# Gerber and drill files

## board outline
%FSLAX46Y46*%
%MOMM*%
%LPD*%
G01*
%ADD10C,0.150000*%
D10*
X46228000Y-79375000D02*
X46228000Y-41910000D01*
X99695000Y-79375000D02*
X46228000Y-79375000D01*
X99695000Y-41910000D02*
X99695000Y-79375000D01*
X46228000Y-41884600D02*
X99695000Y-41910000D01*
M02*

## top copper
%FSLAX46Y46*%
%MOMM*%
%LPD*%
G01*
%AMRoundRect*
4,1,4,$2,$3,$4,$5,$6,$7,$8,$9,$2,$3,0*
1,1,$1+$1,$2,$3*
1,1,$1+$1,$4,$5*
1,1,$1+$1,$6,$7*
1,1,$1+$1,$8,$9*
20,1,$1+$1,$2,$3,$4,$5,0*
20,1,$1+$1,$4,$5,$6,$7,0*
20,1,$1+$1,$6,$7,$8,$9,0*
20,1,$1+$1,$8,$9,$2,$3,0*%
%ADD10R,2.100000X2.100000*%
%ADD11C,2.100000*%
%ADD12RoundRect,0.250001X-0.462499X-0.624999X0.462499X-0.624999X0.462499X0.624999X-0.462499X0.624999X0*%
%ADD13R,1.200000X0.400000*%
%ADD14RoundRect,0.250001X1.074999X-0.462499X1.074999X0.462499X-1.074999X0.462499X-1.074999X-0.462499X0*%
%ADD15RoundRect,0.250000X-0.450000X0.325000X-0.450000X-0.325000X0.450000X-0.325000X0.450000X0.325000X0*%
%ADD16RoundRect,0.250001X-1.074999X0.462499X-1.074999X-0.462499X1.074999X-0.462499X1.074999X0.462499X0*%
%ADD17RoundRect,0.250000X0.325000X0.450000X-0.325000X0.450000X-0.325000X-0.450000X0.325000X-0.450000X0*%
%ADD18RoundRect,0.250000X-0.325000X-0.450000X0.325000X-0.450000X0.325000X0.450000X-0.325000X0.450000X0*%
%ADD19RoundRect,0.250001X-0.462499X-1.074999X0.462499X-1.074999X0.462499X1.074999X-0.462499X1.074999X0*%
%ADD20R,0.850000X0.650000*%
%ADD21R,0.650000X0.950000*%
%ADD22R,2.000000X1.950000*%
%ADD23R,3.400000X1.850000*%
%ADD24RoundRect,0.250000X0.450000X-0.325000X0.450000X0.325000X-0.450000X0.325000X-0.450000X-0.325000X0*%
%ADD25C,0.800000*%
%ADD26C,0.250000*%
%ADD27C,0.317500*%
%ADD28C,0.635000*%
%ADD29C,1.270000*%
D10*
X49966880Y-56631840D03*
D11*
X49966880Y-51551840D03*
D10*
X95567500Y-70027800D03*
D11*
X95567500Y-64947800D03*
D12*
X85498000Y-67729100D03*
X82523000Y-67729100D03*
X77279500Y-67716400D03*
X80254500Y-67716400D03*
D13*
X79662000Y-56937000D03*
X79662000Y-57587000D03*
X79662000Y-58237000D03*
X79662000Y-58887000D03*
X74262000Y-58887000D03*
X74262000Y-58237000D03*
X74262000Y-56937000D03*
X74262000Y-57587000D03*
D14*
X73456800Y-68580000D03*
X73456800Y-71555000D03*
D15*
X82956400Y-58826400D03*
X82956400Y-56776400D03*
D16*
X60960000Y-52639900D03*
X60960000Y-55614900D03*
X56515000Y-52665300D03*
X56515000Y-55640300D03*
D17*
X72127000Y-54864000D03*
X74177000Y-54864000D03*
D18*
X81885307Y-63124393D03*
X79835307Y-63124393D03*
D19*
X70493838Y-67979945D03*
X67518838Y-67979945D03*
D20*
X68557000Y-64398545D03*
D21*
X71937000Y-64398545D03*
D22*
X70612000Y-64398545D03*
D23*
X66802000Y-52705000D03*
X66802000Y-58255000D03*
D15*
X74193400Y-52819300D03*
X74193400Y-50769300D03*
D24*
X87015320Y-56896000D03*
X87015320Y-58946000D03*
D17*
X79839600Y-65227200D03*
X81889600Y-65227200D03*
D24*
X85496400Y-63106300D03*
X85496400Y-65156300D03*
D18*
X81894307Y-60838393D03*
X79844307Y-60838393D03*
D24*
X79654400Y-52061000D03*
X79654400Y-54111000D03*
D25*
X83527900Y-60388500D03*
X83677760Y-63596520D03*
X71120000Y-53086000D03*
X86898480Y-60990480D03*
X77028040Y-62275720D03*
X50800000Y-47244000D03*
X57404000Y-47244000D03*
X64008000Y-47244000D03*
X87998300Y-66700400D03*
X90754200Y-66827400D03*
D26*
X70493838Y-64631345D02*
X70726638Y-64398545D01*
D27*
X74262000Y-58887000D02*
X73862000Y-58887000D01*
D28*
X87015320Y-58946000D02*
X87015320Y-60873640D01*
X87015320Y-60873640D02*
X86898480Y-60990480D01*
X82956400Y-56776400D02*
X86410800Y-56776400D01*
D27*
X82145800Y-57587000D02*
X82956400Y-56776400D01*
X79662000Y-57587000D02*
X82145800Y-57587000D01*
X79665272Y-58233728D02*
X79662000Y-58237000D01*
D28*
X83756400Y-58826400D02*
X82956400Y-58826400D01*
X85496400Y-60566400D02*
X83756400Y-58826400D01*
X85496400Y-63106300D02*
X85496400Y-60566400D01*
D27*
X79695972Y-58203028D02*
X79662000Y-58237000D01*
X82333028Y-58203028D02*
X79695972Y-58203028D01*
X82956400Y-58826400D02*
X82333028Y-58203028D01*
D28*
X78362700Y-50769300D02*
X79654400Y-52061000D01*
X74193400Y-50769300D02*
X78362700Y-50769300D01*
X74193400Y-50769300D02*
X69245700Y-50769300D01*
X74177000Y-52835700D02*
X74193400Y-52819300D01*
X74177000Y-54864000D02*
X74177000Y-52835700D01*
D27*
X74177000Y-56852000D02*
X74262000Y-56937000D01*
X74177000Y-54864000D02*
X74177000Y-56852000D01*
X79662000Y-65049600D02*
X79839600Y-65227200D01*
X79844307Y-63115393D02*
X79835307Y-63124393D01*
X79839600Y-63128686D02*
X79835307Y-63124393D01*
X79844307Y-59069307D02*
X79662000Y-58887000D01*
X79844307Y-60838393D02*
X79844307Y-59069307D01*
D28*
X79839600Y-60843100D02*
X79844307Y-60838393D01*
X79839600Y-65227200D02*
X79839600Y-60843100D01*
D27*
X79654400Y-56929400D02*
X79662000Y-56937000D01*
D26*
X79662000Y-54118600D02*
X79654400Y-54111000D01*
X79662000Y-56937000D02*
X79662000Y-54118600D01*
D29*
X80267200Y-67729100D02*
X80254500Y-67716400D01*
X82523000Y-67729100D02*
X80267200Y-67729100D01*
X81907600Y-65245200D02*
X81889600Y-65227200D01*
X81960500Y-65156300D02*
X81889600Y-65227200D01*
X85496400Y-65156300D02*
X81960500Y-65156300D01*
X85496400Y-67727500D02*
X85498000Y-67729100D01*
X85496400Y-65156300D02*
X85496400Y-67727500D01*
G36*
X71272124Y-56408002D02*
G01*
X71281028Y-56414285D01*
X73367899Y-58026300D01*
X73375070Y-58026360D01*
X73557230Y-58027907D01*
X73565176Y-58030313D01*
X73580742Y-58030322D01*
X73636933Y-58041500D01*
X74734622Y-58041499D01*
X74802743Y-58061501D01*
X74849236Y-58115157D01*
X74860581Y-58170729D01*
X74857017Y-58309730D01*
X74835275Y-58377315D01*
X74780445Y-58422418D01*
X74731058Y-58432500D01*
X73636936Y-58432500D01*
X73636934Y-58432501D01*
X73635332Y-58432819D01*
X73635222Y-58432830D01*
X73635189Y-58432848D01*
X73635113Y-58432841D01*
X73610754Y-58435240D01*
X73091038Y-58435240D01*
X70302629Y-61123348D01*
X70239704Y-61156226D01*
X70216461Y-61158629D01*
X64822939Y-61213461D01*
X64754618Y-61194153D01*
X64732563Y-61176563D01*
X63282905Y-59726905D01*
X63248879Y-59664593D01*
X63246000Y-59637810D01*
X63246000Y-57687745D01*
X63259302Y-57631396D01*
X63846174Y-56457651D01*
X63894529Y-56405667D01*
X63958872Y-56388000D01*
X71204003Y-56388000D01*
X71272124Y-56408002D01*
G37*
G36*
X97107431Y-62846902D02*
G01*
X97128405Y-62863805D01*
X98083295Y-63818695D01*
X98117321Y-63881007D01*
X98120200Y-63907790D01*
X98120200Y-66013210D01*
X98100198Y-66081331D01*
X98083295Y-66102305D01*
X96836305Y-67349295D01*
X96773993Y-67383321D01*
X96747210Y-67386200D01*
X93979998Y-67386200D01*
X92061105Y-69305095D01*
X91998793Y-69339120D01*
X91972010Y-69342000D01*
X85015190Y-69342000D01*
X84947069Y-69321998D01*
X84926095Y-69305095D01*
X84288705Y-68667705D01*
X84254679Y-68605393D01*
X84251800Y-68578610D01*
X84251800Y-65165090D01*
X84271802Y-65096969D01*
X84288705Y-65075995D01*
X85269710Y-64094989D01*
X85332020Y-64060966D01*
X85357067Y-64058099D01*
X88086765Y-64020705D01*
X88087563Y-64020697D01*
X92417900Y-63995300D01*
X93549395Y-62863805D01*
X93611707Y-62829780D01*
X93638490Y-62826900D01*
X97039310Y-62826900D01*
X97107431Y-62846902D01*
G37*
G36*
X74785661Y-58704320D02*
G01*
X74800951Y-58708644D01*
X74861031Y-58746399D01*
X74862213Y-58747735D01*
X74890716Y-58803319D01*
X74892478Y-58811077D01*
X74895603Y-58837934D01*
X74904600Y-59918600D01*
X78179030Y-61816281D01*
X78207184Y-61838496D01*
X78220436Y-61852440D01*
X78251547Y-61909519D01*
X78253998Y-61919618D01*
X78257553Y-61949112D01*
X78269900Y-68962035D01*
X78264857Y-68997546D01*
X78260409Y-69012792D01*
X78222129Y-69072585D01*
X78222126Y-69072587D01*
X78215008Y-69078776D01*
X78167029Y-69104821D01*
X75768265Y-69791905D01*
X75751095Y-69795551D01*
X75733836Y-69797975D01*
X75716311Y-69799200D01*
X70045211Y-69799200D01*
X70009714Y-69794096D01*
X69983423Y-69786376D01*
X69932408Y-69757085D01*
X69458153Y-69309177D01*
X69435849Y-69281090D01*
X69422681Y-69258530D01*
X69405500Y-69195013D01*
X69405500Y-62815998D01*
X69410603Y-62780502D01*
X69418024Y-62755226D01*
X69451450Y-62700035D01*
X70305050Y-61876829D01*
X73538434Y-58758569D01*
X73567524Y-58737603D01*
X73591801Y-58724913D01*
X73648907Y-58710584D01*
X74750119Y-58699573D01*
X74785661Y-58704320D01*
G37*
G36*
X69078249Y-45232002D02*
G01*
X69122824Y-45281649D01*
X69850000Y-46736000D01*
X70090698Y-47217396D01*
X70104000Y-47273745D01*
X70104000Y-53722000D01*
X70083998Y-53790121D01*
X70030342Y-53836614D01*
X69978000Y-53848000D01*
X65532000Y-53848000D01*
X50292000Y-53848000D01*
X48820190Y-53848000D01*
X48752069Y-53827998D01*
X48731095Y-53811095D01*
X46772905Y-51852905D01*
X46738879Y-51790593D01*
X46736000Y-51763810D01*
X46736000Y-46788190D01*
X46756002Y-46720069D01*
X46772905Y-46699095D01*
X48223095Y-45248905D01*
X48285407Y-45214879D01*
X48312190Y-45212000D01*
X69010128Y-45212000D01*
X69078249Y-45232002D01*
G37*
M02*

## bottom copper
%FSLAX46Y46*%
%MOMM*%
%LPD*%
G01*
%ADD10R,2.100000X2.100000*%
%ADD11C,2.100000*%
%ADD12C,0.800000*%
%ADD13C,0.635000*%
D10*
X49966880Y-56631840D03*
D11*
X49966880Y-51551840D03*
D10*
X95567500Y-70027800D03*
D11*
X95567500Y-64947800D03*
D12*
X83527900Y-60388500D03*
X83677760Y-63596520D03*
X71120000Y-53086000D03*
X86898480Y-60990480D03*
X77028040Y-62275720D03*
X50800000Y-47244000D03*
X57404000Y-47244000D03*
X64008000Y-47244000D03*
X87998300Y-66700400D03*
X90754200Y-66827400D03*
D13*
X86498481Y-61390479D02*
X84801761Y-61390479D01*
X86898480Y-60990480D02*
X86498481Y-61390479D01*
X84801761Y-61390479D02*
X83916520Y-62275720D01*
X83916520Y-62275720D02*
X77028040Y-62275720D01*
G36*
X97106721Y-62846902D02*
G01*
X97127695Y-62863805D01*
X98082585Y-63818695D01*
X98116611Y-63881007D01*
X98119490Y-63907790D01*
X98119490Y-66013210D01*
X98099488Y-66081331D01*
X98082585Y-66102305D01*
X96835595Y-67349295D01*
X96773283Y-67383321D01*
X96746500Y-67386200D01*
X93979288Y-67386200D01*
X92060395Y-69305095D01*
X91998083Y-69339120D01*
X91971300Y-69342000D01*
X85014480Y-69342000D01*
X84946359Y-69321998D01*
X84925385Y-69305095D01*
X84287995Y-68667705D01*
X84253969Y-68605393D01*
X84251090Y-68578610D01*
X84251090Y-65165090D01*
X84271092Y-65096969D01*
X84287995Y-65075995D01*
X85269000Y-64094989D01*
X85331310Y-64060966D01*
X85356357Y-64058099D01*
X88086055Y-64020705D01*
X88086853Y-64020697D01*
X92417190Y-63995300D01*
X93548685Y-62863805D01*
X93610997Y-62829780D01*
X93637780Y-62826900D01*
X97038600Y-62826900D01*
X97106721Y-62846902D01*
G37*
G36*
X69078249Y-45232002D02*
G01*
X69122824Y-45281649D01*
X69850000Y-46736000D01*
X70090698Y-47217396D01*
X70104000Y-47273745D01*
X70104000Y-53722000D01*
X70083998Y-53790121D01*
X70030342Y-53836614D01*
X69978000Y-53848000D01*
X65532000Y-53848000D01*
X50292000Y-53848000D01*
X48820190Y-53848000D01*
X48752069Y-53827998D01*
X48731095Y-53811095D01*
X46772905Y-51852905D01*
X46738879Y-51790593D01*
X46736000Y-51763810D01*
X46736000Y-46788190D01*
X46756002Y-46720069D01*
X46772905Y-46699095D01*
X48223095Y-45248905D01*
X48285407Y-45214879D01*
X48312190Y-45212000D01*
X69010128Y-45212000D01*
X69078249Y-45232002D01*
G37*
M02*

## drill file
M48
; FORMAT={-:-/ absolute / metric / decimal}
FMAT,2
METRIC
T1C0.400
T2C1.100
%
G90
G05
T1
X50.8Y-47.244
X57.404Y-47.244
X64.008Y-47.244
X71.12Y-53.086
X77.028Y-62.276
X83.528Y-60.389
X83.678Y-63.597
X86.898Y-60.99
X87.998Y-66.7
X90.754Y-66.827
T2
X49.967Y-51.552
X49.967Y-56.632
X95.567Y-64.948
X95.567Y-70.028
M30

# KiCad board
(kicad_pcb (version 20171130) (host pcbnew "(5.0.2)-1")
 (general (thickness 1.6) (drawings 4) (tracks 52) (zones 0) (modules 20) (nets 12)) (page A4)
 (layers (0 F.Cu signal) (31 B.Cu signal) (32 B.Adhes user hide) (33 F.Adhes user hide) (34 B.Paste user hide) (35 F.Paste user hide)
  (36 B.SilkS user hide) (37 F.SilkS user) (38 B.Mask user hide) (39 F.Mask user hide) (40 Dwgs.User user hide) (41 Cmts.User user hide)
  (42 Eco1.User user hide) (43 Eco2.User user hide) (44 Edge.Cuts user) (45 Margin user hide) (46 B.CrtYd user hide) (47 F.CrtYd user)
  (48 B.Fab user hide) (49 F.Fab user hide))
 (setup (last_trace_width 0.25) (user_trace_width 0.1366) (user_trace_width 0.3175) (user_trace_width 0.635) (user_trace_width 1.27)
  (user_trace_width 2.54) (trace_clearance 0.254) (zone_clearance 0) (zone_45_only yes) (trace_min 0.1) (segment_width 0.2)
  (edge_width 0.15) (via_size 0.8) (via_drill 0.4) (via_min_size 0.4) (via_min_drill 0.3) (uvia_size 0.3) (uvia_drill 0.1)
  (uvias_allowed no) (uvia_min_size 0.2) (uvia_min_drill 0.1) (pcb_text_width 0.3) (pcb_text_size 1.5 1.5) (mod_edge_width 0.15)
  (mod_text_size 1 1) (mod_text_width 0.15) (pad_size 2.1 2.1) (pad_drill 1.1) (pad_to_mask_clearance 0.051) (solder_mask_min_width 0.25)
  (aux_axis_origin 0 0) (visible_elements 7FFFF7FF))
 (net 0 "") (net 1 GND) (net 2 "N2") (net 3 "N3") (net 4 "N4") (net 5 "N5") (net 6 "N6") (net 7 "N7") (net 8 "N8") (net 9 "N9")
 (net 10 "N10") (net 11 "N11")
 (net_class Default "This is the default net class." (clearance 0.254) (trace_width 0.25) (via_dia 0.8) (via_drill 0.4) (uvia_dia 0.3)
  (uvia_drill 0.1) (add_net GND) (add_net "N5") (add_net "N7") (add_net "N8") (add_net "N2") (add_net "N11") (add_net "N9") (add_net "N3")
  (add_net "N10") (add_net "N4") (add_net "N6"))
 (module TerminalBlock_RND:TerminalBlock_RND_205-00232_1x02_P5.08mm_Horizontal (layer F.Cu) (at 49.96688 56.63184 90)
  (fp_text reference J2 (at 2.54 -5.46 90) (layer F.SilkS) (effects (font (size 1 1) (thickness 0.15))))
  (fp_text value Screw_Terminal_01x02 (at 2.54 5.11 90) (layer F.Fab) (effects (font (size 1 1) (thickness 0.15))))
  (pad 1 thru_hole rect (at 0 0 90) (size 2.1 2.1) (drill 1.1) (layers *.Cu *.Mask) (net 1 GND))
  (pad 2 thru_hole circle (at 5.08 0 90) (size 2.1 2.1) (drill 1.1) (layers *.Cu *.Mask) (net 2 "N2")))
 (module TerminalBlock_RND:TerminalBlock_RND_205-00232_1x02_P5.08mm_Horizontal (layer F.Cu) (at 95.5675 70.0278 90)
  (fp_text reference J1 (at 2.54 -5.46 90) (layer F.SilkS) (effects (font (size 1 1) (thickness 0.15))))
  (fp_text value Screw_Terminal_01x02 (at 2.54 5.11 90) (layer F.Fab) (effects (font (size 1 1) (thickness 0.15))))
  (pad 1 thru_hole rect (at 0 0 90) (size 2.1 2.1) (drill 1.1) (layers *.Cu *.Mask) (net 1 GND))
  (pad 2 thru_hole circle (at 5.08 0 90) (size 2.1 2.1) (drill 1.1) (layers *.Cu *.Mask) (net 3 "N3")))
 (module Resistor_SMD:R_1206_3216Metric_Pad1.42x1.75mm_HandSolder (layer F.Cu) (at 84.0105 67.7291)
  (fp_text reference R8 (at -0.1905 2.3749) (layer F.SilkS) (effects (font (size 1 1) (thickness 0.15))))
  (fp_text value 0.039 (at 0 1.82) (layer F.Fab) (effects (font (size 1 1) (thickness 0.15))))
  (pad 2 smd roundrect (at 1.4875 0) (size 1.425 1.75) (layers F.Cu F.Paste F.Mask) (roundrect_rratio 0.175439) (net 3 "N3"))
  (pad 1 smd roundrect (at -1.4875 0) (size 1.425 1.75) (layers F.Cu F.Paste F.Mask) (roundrect_rratio 0.175439) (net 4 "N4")))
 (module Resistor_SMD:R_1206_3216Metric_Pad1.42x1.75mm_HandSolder (layer F.Cu) (at 78.767 67.7164)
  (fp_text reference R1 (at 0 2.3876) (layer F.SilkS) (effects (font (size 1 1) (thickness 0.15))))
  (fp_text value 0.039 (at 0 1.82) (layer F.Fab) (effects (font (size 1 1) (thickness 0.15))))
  (pad 1 smd roundrect (at -1.4875 0) (size 1.425 1.75) (layers F.Cu F.Paste F.Mask) (roundrect_rratio 0.175439) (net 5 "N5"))
  (pad 2 smd roundrect (at 1.4875 0) (size 1.425 1.75) (layers F.Cu F.Paste F.Mask) (roundrect_rratio 0.175439) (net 4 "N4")))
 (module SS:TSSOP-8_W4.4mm (layer F.Cu) (at 76.962 57.912)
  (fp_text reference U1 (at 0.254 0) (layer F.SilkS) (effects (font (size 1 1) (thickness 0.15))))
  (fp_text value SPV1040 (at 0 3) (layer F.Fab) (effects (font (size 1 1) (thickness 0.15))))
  (pad 8 smd rect (at 2.7 -0.975) (size 1.2 0.4) (layers F.Cu F.Paste F.Mask) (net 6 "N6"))
  (pad 7 smd rect (at 2.7 -0.325) (size 1.2 0.4) (layers F.Cu F.Paste F.Mask) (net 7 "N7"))
  (pad 6 smd rect (at 2.7 0.325) (size 1.2 0.4) (layers F.Cu F.Paste F.Mask) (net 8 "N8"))
  (pad 5 smd rect (at 2.7 0.975) (size 1.2 0.4) (layers F.Cu F.Paste F.Mask) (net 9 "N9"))
  (pad 4 smd rect (at -2.7 0.975) (size 1.2 0.4) (layers F.Cu F.Paste F.Mask) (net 5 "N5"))
  (pad 3 smd rect (at -2.7 0.325) (size 1.2 0.4) (layers F.Cu F.Paste F.Mask) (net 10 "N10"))
  (pad 1 smd rect (at -2.7 -0.975) (size 1.2 0.4) (layers F.Cu F.Paste F.Mask) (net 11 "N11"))
  (pad 2 smd rect (at -2.7 -0.325) (size 1.2 0.4) (layers F.Cu F.Paste F.Mask) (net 1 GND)))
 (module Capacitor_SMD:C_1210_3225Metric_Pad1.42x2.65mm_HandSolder (layer F.Cu) (at 73.4568 70.0675 90)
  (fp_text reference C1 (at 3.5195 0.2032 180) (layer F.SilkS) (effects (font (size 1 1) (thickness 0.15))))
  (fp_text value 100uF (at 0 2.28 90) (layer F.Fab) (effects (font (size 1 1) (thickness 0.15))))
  (pad 2 smd roundrect (at 1.4875 0 90) (size 1.425 2.65) (layers F.Cu F.Paste F.Mask) (roundrect_rratio 0.175439) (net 5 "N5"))
  (pad 1 smd roundrect (at -1.4875 0 90) (size 1.425 2.65) (layers F.Cu F.Paste F.Mask) (roundrect_rratio 0.175439) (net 1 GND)))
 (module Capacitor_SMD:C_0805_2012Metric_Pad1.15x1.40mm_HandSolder (layer F.Cu) (at 82.9564 57.8014 270)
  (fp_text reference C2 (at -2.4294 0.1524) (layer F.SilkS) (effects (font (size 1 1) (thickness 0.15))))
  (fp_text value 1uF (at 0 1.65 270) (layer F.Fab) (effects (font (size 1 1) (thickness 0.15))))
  (pad 2 smd roundrect (at 1.025 0 270) (size 1.15 1.4) (layers F.Cu F.Paste F.Mask) (roundrect_rratio 0.217391) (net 8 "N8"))
  (pad 1 smd roundrect (at -1.025 0 270) (size 1.15 1.4) (layers F.Cu F.Paste F.Mask) (roundrect_rratio 0.217391) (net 7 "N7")))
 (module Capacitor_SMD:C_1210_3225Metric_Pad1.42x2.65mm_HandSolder (layer F.Cu) (at 60.96 54.1274 270)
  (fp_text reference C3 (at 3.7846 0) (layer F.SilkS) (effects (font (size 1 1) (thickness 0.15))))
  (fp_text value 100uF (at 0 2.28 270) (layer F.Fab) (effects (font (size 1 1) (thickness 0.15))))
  (pad 1 smd roundrect (at -1.4875 0 270) (size 1.425 2.65) (layers F.Cu F.Paste F.Mask) (roundrect_rratio 0.175439) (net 2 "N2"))
  (pad 2 smd roundrect (at 1.4875 0 270) (size 1.425 2.65) (layers F.Cu F.Paste F.Mask) (roundrect_rratio 0.175439) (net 1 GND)))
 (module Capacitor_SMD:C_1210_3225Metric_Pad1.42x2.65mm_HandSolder (layer F.Cu) (at 56.515 54.1528 270)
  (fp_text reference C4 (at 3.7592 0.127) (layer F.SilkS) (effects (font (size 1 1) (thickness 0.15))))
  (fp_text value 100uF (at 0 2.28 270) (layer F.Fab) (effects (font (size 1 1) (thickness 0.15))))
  (pad 1 smd roundrect (at -1.4875 0 270) (size 1.425 2.65) (layers F.Cu F.Paste F.Mask) (roundrect_rratio 0.175439) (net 2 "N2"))
  (pad 2 smd roundrect (at 1.4875 0 270) (size 1.425 2.65) (layers F.Cu F.Paste F.Mask) (roundrect_rratio 0.175439) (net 1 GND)))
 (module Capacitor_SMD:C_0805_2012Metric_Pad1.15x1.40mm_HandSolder (layer F.Cu) (at 73.152 54.864 180)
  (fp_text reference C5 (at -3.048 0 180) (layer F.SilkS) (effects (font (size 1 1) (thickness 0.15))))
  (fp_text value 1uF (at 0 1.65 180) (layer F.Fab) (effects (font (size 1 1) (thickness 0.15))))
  (pad 2 smd roundrect (at 1.025 0 180) (size 1.15 1.4) (layers F.Cu F.Paste F.Mask) (roundrect_rratio 0.217391) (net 1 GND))
  (pad 1 smd roundrect (at -1.025 0 180) (size 1.15 1.4) (layers F.Cu F.Paste F.Mask) (roundrect_rratio 0.217391) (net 11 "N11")))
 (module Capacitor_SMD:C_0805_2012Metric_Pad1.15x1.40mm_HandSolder (layer F.Cu) (at 80.860307 63.124393)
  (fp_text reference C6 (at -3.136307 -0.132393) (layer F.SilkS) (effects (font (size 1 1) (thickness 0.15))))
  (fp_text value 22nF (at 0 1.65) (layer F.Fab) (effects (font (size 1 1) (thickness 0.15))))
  (pad 2 smd roundrect (at 1.025 0) (size 1.15 1.4) (layers F.Cu F.Paste F.Mask) (roundrect_rratio 0.217391) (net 1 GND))
  (pad 1 smd roundrect (at -1.025 0) (size 1.15 1.4) (layers F.Cu F.Paste F.Mask) (roundrect_rratio 0.217391) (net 9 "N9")))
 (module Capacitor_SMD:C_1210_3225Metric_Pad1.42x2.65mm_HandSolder (layer F.Cu) (at 69.006338 67.979945)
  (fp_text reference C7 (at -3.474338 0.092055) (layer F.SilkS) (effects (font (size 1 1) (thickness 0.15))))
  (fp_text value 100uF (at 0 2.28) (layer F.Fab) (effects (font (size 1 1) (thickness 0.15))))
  (pad 2 smd roundrect (at 1.4875 0) (size 1.425 2.65) (layers F.Cu F.Paste F.Mask) (roundrect_rratio 0.175439) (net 5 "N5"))
  (pad 1 smd roundrect (at -1.4875 0) (size 1.425 2.65) (layers F.Cu F.Paste F.Mask) (roundrect_rratio 0.175439) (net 1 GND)))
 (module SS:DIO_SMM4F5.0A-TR (layer F.Cu) (at 70.197 64.398545 180)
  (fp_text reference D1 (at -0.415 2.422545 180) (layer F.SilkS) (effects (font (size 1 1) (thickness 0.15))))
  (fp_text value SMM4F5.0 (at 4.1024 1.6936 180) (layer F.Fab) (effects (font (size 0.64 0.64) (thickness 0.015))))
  (pad 2 smd rect (at 1.64 0 180) (size 0.85 0.65) (layers F.Cu F.Paste F.Mask) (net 1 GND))
  (pad 1 smd rect (at -1.74 0 180) (size 0.65 0.95) (layers F.Cu F.Paste F.Mask) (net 5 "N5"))
  (pad 1 smd rect (at -0.415 0 180) (size 2 1.95) (layers F.Cu F.Paste F.Mask) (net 5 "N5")))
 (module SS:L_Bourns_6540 (layer F.Cu) (at 66.802 52.705 270)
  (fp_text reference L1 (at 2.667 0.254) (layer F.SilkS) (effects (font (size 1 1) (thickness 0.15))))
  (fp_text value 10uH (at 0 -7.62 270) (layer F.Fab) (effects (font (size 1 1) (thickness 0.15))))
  (pad 1 smd rect (at 0 0 270) (size 1.85 3.4) (layers F.Cu F.Paste F.Mask) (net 2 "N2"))
  (pad 2 smd rect (at 5.55 0 270) (size 1.85 3.4) (layers F.Cu F.Paste F.Mask) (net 10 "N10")))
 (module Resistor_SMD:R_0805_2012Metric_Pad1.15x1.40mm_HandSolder (layer F.Cu) (at 74.1934 51.7943 270)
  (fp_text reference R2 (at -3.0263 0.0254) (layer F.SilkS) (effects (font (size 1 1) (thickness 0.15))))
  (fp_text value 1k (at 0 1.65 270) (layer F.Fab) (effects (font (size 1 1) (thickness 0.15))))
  (pad 2 smd roundrect (at 1.025 0 270) (size 1.15 1.4) (layers F.Cu F.Paste F.Mask) (roundrect_rratio 0.217391) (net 11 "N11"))
  (pad 1 smd roundrect (at -1.025 0 270) (size 1.15 1.4) (layers F.Cu F.Paste F.Mask) (roundrect_rratio 0.217391) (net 2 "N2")))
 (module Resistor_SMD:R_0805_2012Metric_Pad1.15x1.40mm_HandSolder (layer F.Cu) (at 87.01532 57.921 90)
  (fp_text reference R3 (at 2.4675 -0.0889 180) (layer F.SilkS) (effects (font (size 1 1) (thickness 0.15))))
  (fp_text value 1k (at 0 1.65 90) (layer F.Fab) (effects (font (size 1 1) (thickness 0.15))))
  (pad 2 smd roundrect (at 1.025 0 90) (size 1.15 1.4) (layers F.Cu F.Paste F.Mask) (roundrect_rratio 0.217391) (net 7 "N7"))
  (pad 1 smd roundrect (at -1.025 0 90) (size 1.15 1.4) (layers F.Cu F.Paste F.Mask) (roundrect_rratio 0.217391) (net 5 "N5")))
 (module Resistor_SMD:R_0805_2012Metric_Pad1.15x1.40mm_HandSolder (layer F.Cu) (at 80.8646 65.2272 180)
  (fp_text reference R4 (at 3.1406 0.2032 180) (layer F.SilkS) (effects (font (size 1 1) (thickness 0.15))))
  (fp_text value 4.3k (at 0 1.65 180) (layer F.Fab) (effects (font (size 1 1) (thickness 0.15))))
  (pad 2 smd roundrect (at 1.025 0 180) (size 1.15 1.4) (layers F.Cu F.Paste F.Mask) (roundrect_rratio 0.217391) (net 9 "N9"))
  (pad 1 smd roundrect (at -1.025 0 180) (size 1.15 1.4) (layers F.Cu F.Paste F.Mask) (roundrect_rratio 0.217391) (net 3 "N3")))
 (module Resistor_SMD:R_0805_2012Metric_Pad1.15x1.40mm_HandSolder (layer F.Cu) (at 85.4964 64.1313 90)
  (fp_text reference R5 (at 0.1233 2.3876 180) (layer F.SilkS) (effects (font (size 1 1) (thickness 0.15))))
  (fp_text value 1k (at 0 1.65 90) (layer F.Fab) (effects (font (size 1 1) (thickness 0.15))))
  (pad 2 smd roundrect (at 1.025 0 90) (size 1.15 1.4) (layers F.Cu F.Paste F.Mask) (roundrect_rratio 0.217391) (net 8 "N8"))
  (pad 1 smd roundrect (at -1.025 0 90) (size 1.15 1.4) (layers F.Cu F.Paste F.Mask) (roundrect_rratio 0.217391) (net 3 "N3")))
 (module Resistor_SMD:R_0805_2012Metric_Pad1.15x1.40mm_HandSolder (layer F.Cu) (at 80.869307 60.838393)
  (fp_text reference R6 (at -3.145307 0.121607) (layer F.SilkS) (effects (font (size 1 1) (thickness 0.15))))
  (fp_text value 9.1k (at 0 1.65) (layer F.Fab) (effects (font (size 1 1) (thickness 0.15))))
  (pad 2 smd roundrect (at 1.025 0) (size 1.15 1.4) (layers F.Cu F.Paste F.Mask) (roundrect_rratio 0.217391) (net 1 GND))
  (pad 1 smd roundrect (at -1.025 0) (size 1.15 1.4) (layers F.Cu F.Paste F.Mask) (roundrect_rratio 0.217391) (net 9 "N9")))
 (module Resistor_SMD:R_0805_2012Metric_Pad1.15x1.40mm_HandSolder (layer F.Cu) (at 79.6544 53.086 90)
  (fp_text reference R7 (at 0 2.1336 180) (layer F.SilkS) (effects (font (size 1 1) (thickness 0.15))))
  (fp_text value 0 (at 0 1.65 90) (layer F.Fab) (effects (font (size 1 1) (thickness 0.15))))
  (pad 2 smd roundrect (at 1.025 0 90) (size 1.15 1.4) (layers F.Cu F.Paste F.Mask) (roundrect_rratio 0.217391) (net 2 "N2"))
  (pad 1 smd roundrect (at -1.025 0 90) (size 1.15 1.4) (layers F.Cu F.Paste F.Mask) (roundrect_rratio 0.217391) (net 6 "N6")))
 (gr_line (start 46.228 79.375) (end 46.228 41.91) (layer Edge.Cuts) (width 0.15))
 (gr_line (start 99.695 79.375) (end 46.228 79.375) (layer Edge.Cuts) (width 0.15))
 (gr_line (start 99.695 41.91) (end 99.695 79.375) (layer Edge.Cuts) (width 0.15))
 (gr_line (start 46.228 41.8846) (end 99.695 41.91) (layer Edge.Cuts) (width 0.15))
 (via (at 83.5279 60.3885) (size 0.8) (drill 0.4) (layers F.Cu B.Cu) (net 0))
 (via (at 83.67776 63.59652) (size 0.8) (drill 0.4) (layers F.Cu B.Cu) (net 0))
 (via (at 71.12 53.086) (size 0.8) (drill 0.4) (layers F.Cu B.Cu) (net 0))
 (segment (start 70.493838 64.631345) (end 70.726638 64.398545) (width 0.25) (layer F.Cu) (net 5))
 (segment (start 74.262 58.887) (end 73.862 58.887) (width 0.3175) (layer F.Cu) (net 5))
 (via (at 86.89848 60.99048) (size 0.8) (drill 0.4) (layers F.Cu B.Cu) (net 5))
 (segment (start 87.01532 58.946) (end 87.01532 60.87364) (width 0.635) (layer F.Cu) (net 5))
 (segment (start 87.01532 60.87364) (end 86.89848 60.99048) (width 0.635) (layer F.Cu) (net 5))
 (segment (start 86.498481 61.390479) (end 84.801761 61.390479) (width 0.635) (layer B.Cu) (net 5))
 (segment (start 86.89848 60.99048) (end 86.498481 61.390479) (width 0.635) (layer B.Cu) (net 5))
 (segment (start 84.801761 61.390479) (end 83.91652 62.27572) (width 0.635) (layer B.Cu) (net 5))
 (via (at 77.02804 62.27572) (size 0.8) (drill 0.4) (layers F.Cu B.Cu) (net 5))
 (segment (start 83.91652 62.27572) (end 77.02804 62.27572) (width 0.635) (layer B.Cu) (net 5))
 (segment (start 82.9564 56.7764) (end 86.4108 56.7764) (width 0.635) (layer F.Cu) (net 7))
 (segment (start 82.1458 57.587) (end 82.9564 56.7764) (width 0.3175) (layer F.Cu) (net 7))
 (segment (start 79.662 57.587) (end 82.1458 57.587) (width 0.3175) (layer F.Cu) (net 7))
 (segment (start 79.665272 58.233728) (end 79.662 58.237) (width 0.3175) (layer F.Cu) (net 8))
 (segment (start 83.7564 58.8264) (end 82.9564 58.8264) (width 0.635) (layer F.Cu) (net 8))
 (segment (start 85.4964 60.5664) (end 83.7564 58.8264) (width 0.635) (layer F.Cu) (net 8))
 (segment (start 85.4964 63.1063) (end 85.4964 60.5664) (width 0.635) (layer F.Cu) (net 8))
 (segment (start 79.695972 58.203028) (end 79.662 58.237) (width 0.3175) (layer F.Cu) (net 8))
 (segment (start 82.333028 58.203028) (end 79.695972 58.203028) (width 0.3175) (layer F.Cu) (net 8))
 (segment (start 82.9564 58.8264) (end 82.333028 58.203028) (width 0.3175) (layer F.Cu) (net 8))
 (via (at 50.8 47.244) (size 0.8) (drill 0.4) (layers F.Cu B.Cu) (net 2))
 (via (at 57.404 47.244) (size 0.8) (drill 0.4) (layers F.Cu B.Cu) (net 2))
 (via (at 64.008 47.244) (size 0.8) (drill 0.4) (layers F.Cu B.Cu) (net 2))
 (segment (start 78.3627 50.7693) (end 79.6544 52.061) (width 0.635) (layer F.Cu) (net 2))
 (segment (start 74.1934 50.7693) (end 78.3627 50.7693) (width 0.635) (layer F.Cu) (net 2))
 (segment (start 74.1934 50.7693) (end 69.2457 50.7693) (width 0.635) (layer F.Cu) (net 2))
 (segment (start 74.177 52.8357) (end 74.1934 52.8193) (width 0.635) (layer F.Cu) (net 11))
 (segment (start 74.177 54.864) (end 74.177 52.8357) (width 0.635) (layer F.Cu) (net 11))
 (segment (start 74.177 56.852) (end 74.262 56.937) (width 0.3175) (layer F.Cu) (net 11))
 (segment (start 74.177 54.864) (end 74.177 56.852) (width 0.3175) (layer F.Cu) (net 11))
 (segment (start 79.662 65.0496) (end 79.8396 65.2272) (width 0.3175) (layer F.Cu) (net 9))
 (segment (start 79.844307 63.115393) (end 79.835307 63.124393) (width 0.3175) (layer F.Cu) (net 9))
 (segment (start 79.8396 63.128686) (end 79.835307 63.124393) (width 0.3175) (layer F.Cu) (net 9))
 (segment (start 79.844307 59.069307) (end 79.662 58.887) (width 0.3175) (layer F.Cu) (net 9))
 (segment (start 79.844307 60.838393) (end 79.844307 59.069307) (width 0.3175) (layer F.Cu) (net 9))
 (segment (start 79.8396 60.8431) (end 79.844307 60.838393) (width 0.635) (layer F.Cu) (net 9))
 (segment (start 79.8396 65.2272) (end 79.8396 60.8431) (width 0.635) (layer F.Cu) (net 9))
 (segment (start 79.6544 56.9294) (end 79.662 56.937) (width 0.3175) (layer F.Cu) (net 6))
 (segment (start 79.662 54.1186) (end 79.6544 54.111) (width 0.25) (layer F.Cu) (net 6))
 (segment (start 79.662 56.937) (end 79.662 54.1186) (width 0.25) (layer F.Cu) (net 6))
 (segment (start 80.2672 67.7291) (end 80.2545 67.7164) (width 1.27) (layer F.Cu) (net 4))
 (segment (start 82.523 67.7291) (end 80.2672 67.7291) (width 1.27) (layer F.Cu) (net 4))
 (segment (start 81.9076 65.2452) (end 81.8896 65.2272) (width 1.27) (layer F.Cu) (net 3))
 (segment (start 81.9605 65.1563) (end 81.8896 65.2272) (width 1.27) (layer F.Cu) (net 3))
 (segment (start 85.4964 65.1563) (end 81.9605 65.1563) (width 1.27) (layer F.Cu) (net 3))
 (segment (start 85.4964 67.7275) (end 85.498 67.7291) (width 1.27) (layer F.Cu) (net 3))
 (segment (start 85.4964 65.1563) (end 85.4964 67.7275) (width 1.27) (layer F.Cu) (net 3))
 (via (at 87.9983 66.7004) (size 0.8) (drill 0.4) (layers F.Cu B.Cu) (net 3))
 (via (at 90.7542 66.8274) (size 0.8) (drill 0.4) (layers F.Cu B.Cu) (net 3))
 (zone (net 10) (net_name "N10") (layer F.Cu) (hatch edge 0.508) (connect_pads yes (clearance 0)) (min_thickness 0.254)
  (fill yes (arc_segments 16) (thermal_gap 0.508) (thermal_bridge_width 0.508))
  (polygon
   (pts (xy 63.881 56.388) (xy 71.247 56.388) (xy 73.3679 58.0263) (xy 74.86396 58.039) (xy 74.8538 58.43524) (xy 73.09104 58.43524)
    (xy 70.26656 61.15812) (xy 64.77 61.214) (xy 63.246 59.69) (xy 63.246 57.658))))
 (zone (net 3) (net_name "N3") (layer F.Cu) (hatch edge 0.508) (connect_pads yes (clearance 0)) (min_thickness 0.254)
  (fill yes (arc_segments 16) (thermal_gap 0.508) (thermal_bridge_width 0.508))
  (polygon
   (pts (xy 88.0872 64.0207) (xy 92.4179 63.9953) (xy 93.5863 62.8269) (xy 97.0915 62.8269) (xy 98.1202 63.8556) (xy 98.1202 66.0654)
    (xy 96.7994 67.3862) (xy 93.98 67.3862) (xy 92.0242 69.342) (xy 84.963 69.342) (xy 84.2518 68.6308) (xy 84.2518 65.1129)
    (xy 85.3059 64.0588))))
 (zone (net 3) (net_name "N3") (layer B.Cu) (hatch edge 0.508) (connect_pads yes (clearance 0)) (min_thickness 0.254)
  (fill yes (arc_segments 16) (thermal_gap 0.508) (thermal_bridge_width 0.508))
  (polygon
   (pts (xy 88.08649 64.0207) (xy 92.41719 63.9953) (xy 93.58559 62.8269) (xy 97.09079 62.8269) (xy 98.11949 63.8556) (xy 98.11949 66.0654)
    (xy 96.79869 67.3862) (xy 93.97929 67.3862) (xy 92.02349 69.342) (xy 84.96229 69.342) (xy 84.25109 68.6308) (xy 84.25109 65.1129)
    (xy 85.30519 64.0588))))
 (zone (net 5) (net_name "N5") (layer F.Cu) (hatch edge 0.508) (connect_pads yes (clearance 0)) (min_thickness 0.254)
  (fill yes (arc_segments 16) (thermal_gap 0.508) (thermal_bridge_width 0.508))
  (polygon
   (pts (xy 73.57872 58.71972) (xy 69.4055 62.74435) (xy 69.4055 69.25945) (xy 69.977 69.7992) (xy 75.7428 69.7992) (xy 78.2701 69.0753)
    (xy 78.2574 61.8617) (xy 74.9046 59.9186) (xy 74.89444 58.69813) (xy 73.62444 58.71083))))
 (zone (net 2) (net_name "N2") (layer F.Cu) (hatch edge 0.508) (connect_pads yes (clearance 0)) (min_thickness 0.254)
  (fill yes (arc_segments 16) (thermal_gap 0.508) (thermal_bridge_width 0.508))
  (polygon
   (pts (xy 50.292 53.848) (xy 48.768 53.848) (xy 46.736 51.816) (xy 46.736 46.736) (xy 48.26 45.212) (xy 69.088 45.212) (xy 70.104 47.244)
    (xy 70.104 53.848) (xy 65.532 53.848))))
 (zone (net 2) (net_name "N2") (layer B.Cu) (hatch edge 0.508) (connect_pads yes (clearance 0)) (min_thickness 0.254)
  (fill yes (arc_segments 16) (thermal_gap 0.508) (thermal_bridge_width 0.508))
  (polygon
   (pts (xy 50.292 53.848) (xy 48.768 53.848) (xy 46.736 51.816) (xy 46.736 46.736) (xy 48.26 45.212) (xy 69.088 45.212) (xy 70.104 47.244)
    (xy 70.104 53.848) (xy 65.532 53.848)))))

